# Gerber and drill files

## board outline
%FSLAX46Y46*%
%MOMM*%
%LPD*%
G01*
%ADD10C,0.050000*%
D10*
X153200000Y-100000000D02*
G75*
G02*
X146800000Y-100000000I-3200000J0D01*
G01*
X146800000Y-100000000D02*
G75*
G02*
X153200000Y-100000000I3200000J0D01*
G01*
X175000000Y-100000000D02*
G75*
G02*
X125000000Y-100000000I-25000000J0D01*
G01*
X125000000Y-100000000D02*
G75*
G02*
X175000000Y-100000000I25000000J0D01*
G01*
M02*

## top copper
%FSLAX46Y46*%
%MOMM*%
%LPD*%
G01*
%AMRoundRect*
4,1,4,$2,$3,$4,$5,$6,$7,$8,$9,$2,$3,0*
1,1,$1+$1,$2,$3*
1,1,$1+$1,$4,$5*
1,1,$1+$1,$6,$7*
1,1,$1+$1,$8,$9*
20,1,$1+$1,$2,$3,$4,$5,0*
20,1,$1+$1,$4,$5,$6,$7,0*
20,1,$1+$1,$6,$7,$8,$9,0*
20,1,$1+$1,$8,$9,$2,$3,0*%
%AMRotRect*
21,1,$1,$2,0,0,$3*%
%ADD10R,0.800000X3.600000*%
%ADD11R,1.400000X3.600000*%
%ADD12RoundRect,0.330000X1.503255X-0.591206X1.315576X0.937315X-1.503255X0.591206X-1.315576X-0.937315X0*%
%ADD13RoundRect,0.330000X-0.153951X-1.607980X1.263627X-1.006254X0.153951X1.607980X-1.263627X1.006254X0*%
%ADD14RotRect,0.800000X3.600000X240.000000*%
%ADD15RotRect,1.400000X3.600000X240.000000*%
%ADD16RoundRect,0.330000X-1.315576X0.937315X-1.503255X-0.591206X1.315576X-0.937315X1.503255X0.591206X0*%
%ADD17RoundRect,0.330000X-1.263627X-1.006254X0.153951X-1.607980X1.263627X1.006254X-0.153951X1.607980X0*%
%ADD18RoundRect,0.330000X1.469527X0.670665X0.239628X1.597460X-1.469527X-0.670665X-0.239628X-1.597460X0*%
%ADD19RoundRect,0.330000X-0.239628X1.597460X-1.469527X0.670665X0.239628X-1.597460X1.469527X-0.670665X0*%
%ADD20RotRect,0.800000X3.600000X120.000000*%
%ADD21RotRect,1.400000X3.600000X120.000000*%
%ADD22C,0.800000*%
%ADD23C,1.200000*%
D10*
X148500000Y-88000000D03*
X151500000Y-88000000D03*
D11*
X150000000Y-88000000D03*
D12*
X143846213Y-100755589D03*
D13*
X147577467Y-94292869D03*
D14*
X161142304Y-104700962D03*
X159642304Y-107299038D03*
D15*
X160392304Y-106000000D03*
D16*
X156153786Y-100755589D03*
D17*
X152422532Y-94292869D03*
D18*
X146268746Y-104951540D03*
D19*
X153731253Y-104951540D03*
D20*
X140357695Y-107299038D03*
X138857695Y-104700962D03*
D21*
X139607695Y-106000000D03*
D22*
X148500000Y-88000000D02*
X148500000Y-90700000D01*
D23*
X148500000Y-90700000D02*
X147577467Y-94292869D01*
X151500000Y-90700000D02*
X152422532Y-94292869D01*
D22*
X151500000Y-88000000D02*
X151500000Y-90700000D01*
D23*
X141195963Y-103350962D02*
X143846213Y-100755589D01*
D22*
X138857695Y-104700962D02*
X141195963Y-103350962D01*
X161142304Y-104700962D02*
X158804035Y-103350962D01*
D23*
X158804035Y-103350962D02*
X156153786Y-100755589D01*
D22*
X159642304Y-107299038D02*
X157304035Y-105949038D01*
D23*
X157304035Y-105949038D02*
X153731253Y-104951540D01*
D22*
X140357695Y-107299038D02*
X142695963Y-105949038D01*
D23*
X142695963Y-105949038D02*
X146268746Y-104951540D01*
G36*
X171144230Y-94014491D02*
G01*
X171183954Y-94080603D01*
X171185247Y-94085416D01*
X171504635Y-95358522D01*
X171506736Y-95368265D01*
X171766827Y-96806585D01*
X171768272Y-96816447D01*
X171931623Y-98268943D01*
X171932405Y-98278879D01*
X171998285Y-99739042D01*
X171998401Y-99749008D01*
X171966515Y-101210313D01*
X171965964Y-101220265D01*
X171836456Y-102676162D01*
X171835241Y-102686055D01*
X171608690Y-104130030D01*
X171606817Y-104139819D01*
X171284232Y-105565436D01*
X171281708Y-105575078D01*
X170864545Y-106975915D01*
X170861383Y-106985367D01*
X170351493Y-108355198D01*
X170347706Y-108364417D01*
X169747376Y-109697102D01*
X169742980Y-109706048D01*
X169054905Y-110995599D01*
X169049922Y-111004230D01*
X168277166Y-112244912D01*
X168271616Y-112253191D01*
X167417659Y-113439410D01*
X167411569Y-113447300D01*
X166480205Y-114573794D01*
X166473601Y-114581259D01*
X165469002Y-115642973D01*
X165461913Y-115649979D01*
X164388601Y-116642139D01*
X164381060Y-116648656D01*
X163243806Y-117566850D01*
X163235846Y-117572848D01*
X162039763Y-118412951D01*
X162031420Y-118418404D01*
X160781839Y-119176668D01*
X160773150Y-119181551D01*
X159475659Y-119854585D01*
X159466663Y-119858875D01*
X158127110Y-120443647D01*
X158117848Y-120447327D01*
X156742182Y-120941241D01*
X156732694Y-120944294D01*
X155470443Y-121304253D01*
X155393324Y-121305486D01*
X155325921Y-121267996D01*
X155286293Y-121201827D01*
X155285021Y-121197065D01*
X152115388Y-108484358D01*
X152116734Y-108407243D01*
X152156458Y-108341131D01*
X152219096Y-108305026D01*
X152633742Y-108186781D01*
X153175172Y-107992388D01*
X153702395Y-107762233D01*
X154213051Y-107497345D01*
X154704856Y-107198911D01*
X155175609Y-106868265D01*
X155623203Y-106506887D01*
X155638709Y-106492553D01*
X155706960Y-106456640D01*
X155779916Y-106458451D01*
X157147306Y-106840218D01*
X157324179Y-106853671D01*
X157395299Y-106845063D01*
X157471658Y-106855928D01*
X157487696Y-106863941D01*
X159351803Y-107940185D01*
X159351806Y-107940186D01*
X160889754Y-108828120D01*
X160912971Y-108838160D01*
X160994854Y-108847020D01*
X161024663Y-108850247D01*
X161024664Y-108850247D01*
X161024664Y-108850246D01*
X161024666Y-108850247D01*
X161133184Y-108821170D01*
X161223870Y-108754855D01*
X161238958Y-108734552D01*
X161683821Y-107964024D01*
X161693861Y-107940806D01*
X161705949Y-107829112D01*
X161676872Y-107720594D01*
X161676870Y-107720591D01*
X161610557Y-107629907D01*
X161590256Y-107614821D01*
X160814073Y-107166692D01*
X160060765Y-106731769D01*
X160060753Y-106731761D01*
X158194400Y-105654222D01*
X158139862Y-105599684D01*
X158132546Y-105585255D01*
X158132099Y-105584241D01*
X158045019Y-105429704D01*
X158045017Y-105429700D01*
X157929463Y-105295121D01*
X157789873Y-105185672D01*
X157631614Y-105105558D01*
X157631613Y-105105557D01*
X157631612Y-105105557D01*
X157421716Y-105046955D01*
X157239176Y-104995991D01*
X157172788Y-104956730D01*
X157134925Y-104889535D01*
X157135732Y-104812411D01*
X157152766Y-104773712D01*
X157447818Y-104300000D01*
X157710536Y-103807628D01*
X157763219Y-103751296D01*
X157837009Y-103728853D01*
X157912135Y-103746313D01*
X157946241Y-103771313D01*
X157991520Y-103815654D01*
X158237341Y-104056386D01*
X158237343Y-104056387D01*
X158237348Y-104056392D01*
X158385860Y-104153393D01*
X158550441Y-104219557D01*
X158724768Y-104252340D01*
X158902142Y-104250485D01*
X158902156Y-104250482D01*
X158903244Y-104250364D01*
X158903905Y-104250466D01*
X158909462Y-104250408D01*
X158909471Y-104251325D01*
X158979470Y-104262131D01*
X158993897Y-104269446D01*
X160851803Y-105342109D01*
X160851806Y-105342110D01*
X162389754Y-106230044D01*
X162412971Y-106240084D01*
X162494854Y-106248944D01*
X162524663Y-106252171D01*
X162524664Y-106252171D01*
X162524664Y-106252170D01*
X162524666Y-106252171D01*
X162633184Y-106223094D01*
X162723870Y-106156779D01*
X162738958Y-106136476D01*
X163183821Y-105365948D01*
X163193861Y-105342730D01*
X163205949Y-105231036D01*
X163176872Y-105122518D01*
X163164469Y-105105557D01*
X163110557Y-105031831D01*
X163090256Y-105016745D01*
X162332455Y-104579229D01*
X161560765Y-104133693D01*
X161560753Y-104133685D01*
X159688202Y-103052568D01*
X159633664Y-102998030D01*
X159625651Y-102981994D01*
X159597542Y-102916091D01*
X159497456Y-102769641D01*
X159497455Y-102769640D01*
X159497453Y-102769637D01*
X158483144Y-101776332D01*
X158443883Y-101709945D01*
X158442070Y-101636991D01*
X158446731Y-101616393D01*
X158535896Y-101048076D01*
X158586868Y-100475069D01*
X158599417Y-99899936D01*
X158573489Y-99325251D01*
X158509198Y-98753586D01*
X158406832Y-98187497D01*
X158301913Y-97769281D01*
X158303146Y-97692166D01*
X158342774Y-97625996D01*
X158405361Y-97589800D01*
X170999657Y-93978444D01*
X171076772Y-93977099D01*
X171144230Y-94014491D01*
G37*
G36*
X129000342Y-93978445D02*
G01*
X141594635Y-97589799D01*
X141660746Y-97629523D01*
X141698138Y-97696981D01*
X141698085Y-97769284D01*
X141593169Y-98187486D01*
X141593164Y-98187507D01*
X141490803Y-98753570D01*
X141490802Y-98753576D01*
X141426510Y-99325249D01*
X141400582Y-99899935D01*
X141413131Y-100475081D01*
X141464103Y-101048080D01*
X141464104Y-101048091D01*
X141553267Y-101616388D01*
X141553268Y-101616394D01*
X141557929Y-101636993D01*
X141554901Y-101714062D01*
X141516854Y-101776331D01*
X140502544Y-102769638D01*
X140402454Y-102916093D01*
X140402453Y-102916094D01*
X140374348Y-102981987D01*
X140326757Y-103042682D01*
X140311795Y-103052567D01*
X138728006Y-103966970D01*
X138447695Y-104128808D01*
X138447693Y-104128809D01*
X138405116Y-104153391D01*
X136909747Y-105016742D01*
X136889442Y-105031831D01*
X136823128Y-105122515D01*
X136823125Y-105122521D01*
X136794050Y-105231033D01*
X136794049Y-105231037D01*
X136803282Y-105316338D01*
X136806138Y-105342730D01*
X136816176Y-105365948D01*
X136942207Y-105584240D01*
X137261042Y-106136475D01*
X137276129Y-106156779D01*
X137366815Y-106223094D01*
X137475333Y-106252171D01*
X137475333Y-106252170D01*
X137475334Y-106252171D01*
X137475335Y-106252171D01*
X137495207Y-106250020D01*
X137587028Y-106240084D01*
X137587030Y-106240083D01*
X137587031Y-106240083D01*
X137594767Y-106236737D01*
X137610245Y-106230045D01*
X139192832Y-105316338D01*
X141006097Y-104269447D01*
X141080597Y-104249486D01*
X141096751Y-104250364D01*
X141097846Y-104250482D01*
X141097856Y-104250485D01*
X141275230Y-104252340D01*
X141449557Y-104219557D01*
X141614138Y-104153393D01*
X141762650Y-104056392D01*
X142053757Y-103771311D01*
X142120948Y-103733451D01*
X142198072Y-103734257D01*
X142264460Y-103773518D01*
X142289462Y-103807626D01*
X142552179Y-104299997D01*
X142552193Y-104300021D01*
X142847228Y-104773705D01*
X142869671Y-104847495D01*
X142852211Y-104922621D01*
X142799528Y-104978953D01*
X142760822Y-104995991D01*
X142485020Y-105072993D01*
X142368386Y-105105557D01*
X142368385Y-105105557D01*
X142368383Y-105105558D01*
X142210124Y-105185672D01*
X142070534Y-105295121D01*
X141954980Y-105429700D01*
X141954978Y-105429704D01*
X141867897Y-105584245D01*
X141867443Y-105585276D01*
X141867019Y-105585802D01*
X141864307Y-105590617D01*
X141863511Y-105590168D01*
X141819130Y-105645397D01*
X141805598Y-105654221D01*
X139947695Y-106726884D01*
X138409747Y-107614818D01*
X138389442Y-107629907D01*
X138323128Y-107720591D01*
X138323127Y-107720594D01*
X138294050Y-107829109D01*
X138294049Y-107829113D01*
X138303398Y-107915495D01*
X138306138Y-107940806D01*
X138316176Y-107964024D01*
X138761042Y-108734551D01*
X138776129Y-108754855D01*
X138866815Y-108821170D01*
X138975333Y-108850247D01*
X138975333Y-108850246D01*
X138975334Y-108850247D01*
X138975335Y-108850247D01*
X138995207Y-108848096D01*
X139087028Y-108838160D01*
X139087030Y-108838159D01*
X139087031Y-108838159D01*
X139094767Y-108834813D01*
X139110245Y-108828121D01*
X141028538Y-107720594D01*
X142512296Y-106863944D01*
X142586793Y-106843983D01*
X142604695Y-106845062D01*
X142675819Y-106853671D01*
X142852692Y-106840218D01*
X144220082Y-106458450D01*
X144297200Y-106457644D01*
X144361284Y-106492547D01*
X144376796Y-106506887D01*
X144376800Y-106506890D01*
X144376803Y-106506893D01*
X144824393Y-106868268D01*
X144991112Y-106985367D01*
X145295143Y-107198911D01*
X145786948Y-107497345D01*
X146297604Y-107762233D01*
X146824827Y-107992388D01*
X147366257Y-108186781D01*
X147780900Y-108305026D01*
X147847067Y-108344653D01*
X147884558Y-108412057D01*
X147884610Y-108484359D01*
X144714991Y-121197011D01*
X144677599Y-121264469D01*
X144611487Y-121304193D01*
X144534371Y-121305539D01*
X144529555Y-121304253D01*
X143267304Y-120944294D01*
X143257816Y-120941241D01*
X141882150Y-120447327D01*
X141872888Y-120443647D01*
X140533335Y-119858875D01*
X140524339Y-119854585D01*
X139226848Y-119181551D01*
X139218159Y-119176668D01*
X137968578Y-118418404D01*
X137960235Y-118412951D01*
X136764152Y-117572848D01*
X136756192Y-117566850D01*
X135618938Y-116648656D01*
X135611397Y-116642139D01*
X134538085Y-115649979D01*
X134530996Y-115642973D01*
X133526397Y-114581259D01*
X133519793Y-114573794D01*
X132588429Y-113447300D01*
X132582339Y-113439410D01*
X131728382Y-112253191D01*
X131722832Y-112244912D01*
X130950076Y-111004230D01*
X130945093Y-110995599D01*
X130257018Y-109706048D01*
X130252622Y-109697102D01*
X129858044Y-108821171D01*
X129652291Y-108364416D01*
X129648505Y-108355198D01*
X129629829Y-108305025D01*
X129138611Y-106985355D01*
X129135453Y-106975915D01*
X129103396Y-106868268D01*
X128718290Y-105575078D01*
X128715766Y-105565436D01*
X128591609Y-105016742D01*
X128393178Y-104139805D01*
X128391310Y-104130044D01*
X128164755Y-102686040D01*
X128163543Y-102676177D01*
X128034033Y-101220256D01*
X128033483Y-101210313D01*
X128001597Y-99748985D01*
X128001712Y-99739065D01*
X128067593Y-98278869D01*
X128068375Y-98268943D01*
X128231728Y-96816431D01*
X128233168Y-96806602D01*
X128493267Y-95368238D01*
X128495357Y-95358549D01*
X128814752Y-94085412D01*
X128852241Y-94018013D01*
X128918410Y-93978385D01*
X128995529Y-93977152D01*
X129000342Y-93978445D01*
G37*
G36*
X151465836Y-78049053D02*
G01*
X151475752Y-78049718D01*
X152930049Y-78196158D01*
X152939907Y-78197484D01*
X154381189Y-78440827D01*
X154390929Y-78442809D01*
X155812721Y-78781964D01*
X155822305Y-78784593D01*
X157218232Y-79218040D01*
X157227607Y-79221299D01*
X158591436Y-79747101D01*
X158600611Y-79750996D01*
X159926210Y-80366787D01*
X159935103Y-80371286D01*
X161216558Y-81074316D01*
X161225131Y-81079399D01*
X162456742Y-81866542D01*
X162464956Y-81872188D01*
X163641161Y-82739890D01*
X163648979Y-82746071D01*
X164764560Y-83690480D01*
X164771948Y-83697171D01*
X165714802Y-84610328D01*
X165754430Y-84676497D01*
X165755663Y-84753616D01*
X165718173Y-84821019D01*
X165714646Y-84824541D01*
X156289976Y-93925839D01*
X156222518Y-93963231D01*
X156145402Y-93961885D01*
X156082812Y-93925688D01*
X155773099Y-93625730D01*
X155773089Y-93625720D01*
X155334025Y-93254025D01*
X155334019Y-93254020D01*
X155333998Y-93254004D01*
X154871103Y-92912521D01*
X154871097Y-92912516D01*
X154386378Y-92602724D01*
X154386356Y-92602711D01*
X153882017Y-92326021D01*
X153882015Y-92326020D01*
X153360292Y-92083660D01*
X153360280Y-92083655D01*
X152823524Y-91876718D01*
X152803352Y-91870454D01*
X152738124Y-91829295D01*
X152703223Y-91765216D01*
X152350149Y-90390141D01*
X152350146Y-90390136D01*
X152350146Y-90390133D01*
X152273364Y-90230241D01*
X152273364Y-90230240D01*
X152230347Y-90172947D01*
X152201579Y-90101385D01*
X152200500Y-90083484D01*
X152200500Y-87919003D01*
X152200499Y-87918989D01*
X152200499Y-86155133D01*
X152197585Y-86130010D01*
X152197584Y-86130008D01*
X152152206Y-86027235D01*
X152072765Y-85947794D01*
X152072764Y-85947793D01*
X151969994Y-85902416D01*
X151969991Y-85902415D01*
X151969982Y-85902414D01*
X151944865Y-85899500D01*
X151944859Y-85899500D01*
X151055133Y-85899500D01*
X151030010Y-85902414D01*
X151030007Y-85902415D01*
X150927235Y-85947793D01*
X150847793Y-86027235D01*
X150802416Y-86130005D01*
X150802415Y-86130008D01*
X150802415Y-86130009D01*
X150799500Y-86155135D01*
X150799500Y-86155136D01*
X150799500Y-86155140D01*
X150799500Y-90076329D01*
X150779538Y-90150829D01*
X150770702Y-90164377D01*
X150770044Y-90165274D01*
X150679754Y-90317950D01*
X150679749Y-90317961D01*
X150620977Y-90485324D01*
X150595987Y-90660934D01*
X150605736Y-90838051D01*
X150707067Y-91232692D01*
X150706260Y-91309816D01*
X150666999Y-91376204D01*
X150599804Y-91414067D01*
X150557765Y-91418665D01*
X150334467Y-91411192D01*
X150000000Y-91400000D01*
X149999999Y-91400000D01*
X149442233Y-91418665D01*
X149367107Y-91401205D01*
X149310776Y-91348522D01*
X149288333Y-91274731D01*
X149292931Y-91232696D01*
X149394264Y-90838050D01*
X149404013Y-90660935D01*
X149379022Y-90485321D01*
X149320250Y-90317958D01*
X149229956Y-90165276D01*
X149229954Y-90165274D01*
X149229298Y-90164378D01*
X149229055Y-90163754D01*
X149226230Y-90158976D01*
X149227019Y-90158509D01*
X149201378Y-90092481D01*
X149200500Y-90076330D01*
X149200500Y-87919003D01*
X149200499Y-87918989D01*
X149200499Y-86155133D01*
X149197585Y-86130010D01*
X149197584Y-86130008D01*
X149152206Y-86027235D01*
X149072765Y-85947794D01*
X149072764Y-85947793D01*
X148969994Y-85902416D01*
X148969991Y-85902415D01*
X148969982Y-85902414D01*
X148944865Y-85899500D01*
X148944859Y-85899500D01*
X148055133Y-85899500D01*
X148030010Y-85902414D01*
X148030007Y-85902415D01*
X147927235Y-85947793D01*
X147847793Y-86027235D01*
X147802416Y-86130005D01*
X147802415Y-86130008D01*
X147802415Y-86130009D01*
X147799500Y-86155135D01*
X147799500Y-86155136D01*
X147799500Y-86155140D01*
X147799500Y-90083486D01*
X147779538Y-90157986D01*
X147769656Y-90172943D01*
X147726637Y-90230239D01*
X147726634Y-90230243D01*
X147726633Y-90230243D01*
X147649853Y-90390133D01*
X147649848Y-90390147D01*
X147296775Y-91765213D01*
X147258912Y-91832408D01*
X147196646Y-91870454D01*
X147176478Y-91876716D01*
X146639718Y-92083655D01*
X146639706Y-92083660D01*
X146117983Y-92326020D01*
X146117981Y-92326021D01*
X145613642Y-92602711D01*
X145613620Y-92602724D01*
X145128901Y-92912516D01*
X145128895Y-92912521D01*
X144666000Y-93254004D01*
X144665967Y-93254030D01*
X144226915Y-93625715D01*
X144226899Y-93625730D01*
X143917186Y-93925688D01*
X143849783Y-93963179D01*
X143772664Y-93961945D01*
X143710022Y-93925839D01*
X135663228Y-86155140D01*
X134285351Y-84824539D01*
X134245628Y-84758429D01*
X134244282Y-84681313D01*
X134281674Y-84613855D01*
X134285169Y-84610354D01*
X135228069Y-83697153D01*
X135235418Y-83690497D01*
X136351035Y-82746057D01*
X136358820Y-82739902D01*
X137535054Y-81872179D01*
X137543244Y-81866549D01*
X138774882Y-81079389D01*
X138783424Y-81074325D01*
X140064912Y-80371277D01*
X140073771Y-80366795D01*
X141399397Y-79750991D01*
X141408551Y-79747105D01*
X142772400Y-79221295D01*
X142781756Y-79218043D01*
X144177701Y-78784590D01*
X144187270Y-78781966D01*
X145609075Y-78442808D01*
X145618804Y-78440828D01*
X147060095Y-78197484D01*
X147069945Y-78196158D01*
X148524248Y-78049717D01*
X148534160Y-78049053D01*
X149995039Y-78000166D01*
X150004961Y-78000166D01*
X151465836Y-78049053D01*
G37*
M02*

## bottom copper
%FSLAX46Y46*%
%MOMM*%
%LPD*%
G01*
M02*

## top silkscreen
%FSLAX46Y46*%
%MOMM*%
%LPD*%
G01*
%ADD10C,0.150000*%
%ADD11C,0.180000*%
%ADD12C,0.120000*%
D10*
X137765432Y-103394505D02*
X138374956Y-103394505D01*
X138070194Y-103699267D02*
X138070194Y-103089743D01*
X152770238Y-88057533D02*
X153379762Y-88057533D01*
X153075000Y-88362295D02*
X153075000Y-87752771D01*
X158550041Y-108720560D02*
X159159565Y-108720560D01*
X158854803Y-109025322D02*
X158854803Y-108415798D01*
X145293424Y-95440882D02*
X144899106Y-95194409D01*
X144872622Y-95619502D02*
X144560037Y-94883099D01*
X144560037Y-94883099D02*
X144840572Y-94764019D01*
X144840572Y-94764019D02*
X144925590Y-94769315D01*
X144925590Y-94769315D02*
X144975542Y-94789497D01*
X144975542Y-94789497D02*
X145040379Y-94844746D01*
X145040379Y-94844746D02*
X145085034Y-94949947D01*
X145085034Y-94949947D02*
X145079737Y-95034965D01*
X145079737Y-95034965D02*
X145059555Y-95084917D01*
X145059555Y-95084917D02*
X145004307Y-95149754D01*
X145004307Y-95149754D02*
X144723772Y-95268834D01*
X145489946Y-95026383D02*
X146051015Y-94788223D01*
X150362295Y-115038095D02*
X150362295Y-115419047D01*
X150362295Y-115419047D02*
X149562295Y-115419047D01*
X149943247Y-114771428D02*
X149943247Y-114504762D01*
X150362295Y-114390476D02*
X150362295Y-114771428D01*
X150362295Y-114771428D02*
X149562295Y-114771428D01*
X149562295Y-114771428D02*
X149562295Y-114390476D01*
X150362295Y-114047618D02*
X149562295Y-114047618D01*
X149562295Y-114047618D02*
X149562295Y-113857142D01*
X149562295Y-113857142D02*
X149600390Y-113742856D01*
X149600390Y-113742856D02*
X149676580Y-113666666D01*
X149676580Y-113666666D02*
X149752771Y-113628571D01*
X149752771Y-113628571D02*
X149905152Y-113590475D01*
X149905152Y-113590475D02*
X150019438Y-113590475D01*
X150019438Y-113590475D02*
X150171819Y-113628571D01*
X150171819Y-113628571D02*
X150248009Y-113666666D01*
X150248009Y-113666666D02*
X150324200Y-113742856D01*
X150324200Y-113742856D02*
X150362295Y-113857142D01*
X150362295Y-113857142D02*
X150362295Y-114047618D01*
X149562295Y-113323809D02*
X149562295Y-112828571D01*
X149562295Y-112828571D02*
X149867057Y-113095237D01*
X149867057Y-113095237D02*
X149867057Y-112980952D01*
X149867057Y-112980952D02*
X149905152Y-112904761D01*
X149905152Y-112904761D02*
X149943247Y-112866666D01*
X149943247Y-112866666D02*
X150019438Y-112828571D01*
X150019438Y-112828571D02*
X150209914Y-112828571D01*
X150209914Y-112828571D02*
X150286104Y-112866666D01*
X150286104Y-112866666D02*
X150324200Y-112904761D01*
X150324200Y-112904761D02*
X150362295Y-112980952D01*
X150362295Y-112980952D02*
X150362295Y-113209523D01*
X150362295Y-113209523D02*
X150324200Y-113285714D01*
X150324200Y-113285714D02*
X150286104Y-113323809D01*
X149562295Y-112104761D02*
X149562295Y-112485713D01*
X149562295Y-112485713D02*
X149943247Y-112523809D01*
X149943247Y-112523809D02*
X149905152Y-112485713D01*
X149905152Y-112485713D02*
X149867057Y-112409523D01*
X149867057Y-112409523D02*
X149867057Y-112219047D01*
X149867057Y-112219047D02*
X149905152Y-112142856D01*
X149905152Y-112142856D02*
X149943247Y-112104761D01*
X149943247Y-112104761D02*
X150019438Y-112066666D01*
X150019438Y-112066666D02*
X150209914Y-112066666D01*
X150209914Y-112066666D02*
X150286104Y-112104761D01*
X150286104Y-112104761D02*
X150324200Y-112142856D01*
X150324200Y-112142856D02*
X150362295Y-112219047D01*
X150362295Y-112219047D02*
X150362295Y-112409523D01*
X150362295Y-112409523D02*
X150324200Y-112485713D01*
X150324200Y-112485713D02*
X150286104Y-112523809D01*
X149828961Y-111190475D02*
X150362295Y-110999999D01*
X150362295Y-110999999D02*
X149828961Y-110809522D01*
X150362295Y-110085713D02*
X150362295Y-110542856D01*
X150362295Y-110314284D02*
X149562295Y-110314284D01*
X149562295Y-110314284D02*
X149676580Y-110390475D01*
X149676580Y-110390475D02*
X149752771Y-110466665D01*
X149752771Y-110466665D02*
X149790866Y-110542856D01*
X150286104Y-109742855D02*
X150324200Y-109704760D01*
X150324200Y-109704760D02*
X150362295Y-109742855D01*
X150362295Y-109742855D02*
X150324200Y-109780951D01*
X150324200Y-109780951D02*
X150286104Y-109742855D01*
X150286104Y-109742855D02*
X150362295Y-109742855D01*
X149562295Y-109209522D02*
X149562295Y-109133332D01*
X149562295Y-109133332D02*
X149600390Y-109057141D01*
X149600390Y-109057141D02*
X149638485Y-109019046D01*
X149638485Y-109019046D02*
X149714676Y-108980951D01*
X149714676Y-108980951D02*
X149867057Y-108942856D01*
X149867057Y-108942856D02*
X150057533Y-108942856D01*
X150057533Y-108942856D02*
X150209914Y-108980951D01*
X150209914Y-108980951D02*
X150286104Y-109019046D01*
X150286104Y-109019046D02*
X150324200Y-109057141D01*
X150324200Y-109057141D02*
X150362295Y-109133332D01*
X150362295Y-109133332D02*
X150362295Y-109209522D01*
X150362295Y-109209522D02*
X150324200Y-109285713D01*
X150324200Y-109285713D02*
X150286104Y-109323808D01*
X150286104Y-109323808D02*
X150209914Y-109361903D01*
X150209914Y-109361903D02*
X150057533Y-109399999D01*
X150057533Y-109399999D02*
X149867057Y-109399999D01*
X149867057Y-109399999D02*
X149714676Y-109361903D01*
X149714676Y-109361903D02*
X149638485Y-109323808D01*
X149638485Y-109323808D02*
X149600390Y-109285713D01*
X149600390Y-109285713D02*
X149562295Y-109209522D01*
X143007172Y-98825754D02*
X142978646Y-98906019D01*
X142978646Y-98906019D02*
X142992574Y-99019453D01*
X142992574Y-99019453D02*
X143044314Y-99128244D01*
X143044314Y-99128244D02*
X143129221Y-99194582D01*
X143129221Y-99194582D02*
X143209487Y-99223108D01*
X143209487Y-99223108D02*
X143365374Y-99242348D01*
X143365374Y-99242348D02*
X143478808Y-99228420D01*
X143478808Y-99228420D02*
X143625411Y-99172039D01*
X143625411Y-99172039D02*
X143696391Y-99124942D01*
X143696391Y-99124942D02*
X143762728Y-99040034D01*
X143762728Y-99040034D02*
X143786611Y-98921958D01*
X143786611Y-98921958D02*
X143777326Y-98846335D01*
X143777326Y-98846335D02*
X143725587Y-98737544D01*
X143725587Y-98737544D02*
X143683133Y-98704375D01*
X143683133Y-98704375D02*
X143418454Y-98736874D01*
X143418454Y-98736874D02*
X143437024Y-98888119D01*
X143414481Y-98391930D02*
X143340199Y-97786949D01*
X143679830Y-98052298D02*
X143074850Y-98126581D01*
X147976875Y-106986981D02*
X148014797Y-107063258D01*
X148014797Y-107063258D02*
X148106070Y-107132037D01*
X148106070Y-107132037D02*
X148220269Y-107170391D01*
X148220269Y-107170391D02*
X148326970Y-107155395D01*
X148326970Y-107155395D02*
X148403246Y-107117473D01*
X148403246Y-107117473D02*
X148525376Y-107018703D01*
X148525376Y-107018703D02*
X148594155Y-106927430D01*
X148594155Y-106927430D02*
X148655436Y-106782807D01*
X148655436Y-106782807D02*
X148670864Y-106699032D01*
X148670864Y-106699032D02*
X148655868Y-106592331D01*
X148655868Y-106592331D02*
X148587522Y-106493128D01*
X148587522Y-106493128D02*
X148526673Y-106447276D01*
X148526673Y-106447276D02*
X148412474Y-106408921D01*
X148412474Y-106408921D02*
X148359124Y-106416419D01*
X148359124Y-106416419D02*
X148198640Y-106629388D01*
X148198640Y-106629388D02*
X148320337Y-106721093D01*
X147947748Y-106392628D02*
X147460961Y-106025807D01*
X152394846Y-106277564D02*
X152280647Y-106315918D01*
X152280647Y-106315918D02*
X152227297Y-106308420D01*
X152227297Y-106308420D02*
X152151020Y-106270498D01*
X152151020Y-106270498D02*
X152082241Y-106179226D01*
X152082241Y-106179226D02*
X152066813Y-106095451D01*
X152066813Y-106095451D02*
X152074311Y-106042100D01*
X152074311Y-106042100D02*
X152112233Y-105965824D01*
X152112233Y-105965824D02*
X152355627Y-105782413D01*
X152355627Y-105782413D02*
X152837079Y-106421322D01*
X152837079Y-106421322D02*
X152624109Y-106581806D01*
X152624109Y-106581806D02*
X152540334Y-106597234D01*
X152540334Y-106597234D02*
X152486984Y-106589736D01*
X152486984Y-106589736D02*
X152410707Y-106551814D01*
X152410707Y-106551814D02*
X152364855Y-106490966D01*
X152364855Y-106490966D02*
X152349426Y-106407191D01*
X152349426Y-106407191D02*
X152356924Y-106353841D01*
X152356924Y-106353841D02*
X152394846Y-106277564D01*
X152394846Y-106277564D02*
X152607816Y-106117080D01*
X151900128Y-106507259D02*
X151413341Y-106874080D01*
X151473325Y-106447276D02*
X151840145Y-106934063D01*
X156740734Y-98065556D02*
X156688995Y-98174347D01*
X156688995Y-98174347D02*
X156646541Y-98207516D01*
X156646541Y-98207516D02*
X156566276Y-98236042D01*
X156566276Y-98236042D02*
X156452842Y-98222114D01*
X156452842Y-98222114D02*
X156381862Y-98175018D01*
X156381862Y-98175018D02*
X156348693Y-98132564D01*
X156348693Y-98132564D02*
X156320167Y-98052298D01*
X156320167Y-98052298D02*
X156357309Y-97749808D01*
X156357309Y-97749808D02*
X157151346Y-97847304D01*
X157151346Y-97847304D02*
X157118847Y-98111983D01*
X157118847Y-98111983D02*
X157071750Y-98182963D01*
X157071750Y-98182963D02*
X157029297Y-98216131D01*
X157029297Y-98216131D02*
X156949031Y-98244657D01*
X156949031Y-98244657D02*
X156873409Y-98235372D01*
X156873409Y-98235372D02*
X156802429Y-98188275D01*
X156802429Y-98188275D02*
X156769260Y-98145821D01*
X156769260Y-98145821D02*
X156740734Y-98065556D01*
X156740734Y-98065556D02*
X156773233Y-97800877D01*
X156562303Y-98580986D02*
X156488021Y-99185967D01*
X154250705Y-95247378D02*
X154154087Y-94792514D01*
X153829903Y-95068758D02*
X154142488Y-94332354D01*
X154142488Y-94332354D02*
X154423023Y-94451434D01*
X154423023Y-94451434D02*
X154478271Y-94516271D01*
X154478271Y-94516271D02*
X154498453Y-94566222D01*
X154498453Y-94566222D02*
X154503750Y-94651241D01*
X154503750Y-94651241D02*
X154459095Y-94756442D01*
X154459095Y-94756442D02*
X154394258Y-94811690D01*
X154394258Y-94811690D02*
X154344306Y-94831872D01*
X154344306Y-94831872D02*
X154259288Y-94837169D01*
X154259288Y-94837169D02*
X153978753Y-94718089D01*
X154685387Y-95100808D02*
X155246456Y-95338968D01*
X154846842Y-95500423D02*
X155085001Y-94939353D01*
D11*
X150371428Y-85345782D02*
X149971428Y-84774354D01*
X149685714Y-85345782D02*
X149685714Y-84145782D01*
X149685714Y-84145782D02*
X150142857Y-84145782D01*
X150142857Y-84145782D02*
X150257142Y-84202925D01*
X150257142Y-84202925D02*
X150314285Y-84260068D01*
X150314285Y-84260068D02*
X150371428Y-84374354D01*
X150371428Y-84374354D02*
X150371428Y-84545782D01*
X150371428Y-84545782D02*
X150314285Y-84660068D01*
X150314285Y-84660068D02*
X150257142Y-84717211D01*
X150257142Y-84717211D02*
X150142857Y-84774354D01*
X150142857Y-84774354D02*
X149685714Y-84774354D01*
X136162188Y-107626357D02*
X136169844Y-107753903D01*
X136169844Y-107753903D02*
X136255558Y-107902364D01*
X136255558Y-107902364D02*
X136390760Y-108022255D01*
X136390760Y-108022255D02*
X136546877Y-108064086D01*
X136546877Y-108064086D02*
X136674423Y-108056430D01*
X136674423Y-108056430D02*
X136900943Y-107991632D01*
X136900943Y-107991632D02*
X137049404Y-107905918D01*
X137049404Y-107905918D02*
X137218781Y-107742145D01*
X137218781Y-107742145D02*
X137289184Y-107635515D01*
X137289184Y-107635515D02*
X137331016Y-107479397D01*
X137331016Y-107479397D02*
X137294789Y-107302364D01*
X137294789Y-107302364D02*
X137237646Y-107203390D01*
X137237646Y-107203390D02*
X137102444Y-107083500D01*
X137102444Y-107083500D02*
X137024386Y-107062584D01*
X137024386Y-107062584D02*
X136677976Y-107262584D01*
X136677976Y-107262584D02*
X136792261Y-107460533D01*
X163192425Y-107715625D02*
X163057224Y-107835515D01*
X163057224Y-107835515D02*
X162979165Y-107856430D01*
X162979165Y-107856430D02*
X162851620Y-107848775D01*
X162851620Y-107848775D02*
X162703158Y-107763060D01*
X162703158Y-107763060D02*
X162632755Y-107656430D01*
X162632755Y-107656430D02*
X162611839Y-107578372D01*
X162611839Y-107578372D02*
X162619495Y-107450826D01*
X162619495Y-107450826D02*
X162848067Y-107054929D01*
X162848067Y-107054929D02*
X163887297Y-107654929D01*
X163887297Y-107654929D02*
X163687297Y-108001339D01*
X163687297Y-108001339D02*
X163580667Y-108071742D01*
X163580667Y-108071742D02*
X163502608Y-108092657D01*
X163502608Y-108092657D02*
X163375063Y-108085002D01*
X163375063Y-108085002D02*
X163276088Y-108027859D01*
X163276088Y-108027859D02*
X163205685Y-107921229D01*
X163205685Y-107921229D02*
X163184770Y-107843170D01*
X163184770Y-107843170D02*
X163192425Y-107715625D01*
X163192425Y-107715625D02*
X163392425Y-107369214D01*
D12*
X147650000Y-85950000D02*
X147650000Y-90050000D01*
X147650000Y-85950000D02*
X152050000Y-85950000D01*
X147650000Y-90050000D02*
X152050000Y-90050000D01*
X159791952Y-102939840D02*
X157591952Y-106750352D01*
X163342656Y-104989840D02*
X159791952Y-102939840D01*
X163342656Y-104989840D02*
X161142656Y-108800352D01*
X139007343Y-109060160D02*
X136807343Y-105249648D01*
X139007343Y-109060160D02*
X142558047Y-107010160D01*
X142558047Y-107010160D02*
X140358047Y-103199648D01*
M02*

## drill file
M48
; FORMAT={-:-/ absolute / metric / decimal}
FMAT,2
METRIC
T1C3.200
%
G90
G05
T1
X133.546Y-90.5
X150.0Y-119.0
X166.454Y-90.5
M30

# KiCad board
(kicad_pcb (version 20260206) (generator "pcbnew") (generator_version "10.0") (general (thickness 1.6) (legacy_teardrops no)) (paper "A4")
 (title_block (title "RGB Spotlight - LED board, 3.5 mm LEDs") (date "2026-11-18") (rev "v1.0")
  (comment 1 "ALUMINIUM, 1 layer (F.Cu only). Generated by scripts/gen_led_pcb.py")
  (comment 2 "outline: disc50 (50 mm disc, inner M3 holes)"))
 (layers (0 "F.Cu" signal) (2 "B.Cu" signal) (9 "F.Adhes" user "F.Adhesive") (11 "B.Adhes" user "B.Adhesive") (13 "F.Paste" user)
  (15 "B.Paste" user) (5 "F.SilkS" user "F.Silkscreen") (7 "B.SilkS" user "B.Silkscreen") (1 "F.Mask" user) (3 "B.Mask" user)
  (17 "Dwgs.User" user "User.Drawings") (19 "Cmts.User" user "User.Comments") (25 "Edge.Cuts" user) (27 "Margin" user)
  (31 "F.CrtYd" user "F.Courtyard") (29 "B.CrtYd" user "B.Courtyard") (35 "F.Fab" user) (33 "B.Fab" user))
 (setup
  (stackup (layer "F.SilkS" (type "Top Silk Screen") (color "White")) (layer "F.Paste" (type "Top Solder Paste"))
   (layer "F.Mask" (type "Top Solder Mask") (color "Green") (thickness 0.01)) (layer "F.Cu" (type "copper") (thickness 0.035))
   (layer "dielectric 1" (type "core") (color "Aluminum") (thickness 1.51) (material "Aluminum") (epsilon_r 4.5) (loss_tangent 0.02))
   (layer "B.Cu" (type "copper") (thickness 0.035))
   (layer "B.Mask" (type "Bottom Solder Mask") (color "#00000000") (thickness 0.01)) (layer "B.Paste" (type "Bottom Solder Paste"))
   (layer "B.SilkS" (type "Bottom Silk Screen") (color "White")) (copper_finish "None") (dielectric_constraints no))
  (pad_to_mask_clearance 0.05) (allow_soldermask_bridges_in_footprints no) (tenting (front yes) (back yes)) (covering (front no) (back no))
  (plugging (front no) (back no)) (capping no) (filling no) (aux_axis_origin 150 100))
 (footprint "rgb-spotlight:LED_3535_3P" (layer "F.Cu") (at 150 88)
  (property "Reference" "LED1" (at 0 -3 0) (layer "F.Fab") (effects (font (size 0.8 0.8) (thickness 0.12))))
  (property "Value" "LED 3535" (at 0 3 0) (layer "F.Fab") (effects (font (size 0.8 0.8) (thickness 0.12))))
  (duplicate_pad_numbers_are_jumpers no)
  (fp_line (start -2.35 -2.05) (end -2.35 2.05) (stroke (width 0.12) (type solid)) (layer "F.SilkS"))
  (fp_line (start -2.35 -2.05) (end 2.05 -2.05) (stroke (width 0.12) (type solid)) (layer "F.SilkS"))
  (fp_line (start -2.35 2.05) (end 2.05 2.05) (stroke (width 0.12) (type solid)) (layer "F.SilkS"))
  (pad "1" smd rect (at -1.5 0) (size 0.8 3.6) (layers "F.Cu" "F.Mask" "F.Paste") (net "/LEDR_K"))
  (pad "2" smd rect (at 1.5 0) (size 0.8 3.6) (layers "F.Cu" "F.Mask" "F.Paste") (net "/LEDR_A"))
  (pad "3" smd rect (at 0 0) (size 1.4 3.6) (layers "F.Cu" "F.Mask" "F.Paste") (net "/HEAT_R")))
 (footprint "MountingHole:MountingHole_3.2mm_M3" (layer "F.Cu") (at 166.454482 90.5)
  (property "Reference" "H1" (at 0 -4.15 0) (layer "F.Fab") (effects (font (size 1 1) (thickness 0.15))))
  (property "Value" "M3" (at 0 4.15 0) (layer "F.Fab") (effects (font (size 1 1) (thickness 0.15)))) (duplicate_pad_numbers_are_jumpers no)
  (pad "" np_thru_hole circle (at 0 0) (size 3.2 3.2) (drill 3.2) (layers "*.Cu" "*.Mask")))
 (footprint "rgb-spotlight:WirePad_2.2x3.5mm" (layer "F.Cu") (at 143.846213 100.755589 97)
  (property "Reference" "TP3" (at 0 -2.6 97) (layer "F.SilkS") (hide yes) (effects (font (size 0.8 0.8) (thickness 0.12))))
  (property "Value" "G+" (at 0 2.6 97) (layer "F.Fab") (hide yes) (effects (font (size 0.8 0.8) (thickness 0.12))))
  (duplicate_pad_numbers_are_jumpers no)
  (pad "1" smd roundrect (at 0 0 97) (size 2.2 3.5) (layers "F.Cu" "F.Mask") (roundrect_rratio 0.15) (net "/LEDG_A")))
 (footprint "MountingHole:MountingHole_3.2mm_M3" (layer "F.Cu") (at 150 119)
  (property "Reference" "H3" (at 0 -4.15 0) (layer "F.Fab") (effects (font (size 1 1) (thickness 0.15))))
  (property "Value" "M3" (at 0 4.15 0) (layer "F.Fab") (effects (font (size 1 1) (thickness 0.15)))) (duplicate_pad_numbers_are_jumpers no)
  (pad "" np_thru_hole circle (at 0 0) (size 3.2 3.2) (drill 3.2) (layers "*.Cu" "*.Mask")))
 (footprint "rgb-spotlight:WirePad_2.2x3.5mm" (layer "F.Cu") (at 147.577467 94.292869 23)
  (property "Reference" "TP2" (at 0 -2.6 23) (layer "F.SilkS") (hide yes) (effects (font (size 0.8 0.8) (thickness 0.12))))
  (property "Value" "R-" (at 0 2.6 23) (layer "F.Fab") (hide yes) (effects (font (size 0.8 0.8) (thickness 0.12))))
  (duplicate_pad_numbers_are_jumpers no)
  (pad "1" smd roundrect (at 0 0 23) (size 2.2 3.5) (layers "F.Cu" "F.Mask") (roundrect_rratio 0.15) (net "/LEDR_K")))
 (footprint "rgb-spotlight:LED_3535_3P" (layer "F.Cu") (at 160.392304 106 -120)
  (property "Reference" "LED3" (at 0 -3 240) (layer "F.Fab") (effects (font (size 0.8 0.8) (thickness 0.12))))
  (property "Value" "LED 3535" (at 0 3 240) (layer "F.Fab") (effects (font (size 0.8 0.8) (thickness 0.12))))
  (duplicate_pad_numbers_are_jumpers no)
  (fp_line (start -2.35 2.05) (end 2.05 2.05) (stroke (width 0.12) (type solid)) (layer "F.SilkS"))
  (fp_line (start -2.35 -2.05) (end -2.35 2.05) (stroke (width 0.12) (type solid)) (layer "F.SilkS"))
  (fp_line (start -2.35 -2.05) (end 2.05 -2.05) (stroke (width 0.12) (type solid)) (layer "F.SilkS"))
  (pad "1" smd rect (at -1.5 0 240) (size 0.8 3.6) (layers "F.Cu" "F.Mask" "F.Paste") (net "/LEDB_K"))
  (pad "2" smd rect (at 1.5 0 240) (size 0.8 3.6) (layers "F.Cu" "F.Mask" "F.Paste") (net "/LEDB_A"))
  (pad "3" smd rect (at 0 0 240) (size 1.4 3.6) (layers "F.Cu" "F.Mask" "F.Paste") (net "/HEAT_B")))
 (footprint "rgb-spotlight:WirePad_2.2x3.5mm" (layer "F.Cu") (at 156.153786 100.755589 -97)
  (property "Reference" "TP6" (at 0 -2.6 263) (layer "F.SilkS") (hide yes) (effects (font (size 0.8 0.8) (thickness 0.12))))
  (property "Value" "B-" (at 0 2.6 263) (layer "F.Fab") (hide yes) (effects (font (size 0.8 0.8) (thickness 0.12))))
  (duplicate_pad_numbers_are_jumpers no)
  (pad "1" smd roundrect (at 0 0 263) (size 2.2 3.5) (layers "F.Cu" "F.Mask") (roundrect_rratio 0.15) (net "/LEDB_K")))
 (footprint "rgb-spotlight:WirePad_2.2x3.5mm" (layer "F.Cu") (at 152.422532 94.292869 -23)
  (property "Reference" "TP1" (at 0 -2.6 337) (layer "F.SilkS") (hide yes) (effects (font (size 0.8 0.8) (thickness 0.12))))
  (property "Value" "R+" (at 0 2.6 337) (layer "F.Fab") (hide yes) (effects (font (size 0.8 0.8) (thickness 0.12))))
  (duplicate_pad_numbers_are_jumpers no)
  (pad "1" smd roundrect (at 0 0 337) (size 2.2 3.5) (layers "F.Cu" "F.Mask") (roundrect_rratio 0.15) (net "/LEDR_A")))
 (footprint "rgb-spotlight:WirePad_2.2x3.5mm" (layer "F.Cu") (at 146.268746 104.95154 143)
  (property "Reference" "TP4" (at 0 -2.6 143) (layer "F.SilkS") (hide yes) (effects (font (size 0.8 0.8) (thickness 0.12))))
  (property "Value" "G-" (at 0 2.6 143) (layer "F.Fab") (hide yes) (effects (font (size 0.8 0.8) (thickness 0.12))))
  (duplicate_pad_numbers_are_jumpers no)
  (pad "1" smd roundrect (at 0 0 143) (size 2.2 3.5) (layers "F.Cu" "F.Mask") (roundrect_rratio 0.15) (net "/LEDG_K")))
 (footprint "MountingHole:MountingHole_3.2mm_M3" (layer "F.Cu") (at 133.545517 90.5)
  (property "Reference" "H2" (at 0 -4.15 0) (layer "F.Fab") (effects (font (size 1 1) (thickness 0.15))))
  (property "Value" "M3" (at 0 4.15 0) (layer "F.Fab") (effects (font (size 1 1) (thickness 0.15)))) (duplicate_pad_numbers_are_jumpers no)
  (pad "" np_thru_hole circle (at 0 0) (size 3.2 3.2) (drill 3.2) (layers "*.Cu" "*.Mask")))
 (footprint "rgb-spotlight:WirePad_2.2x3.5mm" (layer "F.Cu") (at 153.731253 104.95154 -143)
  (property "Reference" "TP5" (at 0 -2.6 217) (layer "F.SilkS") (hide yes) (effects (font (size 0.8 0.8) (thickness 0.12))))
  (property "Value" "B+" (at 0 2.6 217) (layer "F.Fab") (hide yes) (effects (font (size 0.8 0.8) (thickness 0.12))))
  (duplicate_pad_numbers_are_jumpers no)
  (pad "1" smd roundrect (at 0 0 217) (size 2.2 3.5) (layers "F.Cu" "F.Mask") (roundrect_rratio 0.15) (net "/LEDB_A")))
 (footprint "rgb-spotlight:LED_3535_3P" (layer "F.Cu") (at 139.607695 106 120)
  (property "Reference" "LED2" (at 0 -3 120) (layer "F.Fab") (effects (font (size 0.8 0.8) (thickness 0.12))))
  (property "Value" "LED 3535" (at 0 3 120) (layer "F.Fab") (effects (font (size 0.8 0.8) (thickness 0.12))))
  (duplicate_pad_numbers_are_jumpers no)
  (fp_line (start -2.35 -2.05) (end 2.05 -2.05) (stroke (width 0.12) (type solid)) (layer "F.SilkS"))
  (fp_line (start -2.35 -2.05) (end -2.35 2.05) (stroke (width 0.12) (type solid)) (layer "F.SilkS"))
  (fp_line (start -2.35 2.05) (end 2.05 2.05) (stroke (width 0.12) (type solid)) (layer "F.SilkS"))
  (pad "1" smd rect (at -1.5 0 120) (size 0.8 3.6) (layers "F.Cu" "F.Mask" "F.Paste") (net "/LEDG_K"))
  (pad "2" smd rect (at 1.5 0 120) (size 0.8 3.6) (layers "F.Cu" "F.Mask" "F.Paste") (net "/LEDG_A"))
  (pad "3" smd rect (at 0 0 120) (size 1.4 3.6) (layers "F.Cu" "F.Mask" "F.Paste") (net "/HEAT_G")))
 (gr_circle (center 150 100) (end 153.2 100) (stroke (width 0.05) (type default)) (fill no) (layer "Edge.Cuts"))
 (gr_circle (center 150 100) (end 175 100) (stroke (width 0.05) (type default)) (fill no) (layer "Edge.Cuts"))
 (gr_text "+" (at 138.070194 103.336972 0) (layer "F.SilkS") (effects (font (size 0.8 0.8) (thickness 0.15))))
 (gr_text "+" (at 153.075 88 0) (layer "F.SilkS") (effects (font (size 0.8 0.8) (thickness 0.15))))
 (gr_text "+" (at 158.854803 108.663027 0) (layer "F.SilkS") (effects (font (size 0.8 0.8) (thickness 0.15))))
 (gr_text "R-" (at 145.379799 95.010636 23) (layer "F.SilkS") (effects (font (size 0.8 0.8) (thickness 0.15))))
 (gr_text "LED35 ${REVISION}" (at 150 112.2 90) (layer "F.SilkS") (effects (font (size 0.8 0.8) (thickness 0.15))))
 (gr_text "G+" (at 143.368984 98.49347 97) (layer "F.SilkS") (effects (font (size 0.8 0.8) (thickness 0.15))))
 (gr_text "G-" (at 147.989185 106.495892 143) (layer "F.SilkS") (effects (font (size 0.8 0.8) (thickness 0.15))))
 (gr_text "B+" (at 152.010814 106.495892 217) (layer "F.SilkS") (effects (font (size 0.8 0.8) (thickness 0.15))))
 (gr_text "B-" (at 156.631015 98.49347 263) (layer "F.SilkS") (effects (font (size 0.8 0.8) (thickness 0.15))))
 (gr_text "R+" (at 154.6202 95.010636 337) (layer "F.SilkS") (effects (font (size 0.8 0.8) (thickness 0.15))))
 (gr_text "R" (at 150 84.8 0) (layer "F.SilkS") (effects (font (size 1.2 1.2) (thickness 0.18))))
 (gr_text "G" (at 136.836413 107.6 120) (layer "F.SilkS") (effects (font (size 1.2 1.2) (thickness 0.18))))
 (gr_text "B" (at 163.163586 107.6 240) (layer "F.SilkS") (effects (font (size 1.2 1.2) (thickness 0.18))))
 (segment (start 148.5 88) (end 148.5 90.7) (width 0.8) (layer "F.Cu") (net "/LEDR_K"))
 (segment (start 148.5 90.7) (end 147.577467 94.292869) (width 1.2) (layer "F.Cu") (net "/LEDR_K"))
 (segment (start 151.5 90.7) (end 152.422532 94.292869) (width 1.2) (layer "F.Cu") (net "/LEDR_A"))
 (segment (start 151.5 88) (end 151.5 90.7) (width 0.8) (layer "F.Cu") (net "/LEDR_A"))
 (segment (start 141.195963 103.350962) (end 143.846213 100.755589) (width 1.2) (layer "F.Cu") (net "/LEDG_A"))
 (segment (start 138.857695 104.700962) (end 141.195963 103.350962) (width 0.8) (layer "F.Cu") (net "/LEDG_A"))
 (segment (start 161.142304 104.700962) (end 158.804035 103.350962) (width 0.8) (layer "F.Cu") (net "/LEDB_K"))
 (segment (start 158.804035 103.350962) (end 156.153786 100.755589) (width 1.2) (layer "F.Cu") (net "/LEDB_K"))
 (segment (start 159.642304 107.299038) (end 157.304035 105.949038) (width 0.8) (layer "F.Cu") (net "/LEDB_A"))
 (segment (start 157.304035 105.949038) (end 153.731253 104.95154) (width 1.2) (layer "F.Cu") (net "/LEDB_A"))
 (segment (start 140.357695 107.299038) (end 142.695963 105.949038) (width 0.8) (layer "F.Cu") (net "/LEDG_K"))
 (segment (start 142.695963 105.949038) (end 146.268746 104.95154) (width 1.2) (layer "F.Cu") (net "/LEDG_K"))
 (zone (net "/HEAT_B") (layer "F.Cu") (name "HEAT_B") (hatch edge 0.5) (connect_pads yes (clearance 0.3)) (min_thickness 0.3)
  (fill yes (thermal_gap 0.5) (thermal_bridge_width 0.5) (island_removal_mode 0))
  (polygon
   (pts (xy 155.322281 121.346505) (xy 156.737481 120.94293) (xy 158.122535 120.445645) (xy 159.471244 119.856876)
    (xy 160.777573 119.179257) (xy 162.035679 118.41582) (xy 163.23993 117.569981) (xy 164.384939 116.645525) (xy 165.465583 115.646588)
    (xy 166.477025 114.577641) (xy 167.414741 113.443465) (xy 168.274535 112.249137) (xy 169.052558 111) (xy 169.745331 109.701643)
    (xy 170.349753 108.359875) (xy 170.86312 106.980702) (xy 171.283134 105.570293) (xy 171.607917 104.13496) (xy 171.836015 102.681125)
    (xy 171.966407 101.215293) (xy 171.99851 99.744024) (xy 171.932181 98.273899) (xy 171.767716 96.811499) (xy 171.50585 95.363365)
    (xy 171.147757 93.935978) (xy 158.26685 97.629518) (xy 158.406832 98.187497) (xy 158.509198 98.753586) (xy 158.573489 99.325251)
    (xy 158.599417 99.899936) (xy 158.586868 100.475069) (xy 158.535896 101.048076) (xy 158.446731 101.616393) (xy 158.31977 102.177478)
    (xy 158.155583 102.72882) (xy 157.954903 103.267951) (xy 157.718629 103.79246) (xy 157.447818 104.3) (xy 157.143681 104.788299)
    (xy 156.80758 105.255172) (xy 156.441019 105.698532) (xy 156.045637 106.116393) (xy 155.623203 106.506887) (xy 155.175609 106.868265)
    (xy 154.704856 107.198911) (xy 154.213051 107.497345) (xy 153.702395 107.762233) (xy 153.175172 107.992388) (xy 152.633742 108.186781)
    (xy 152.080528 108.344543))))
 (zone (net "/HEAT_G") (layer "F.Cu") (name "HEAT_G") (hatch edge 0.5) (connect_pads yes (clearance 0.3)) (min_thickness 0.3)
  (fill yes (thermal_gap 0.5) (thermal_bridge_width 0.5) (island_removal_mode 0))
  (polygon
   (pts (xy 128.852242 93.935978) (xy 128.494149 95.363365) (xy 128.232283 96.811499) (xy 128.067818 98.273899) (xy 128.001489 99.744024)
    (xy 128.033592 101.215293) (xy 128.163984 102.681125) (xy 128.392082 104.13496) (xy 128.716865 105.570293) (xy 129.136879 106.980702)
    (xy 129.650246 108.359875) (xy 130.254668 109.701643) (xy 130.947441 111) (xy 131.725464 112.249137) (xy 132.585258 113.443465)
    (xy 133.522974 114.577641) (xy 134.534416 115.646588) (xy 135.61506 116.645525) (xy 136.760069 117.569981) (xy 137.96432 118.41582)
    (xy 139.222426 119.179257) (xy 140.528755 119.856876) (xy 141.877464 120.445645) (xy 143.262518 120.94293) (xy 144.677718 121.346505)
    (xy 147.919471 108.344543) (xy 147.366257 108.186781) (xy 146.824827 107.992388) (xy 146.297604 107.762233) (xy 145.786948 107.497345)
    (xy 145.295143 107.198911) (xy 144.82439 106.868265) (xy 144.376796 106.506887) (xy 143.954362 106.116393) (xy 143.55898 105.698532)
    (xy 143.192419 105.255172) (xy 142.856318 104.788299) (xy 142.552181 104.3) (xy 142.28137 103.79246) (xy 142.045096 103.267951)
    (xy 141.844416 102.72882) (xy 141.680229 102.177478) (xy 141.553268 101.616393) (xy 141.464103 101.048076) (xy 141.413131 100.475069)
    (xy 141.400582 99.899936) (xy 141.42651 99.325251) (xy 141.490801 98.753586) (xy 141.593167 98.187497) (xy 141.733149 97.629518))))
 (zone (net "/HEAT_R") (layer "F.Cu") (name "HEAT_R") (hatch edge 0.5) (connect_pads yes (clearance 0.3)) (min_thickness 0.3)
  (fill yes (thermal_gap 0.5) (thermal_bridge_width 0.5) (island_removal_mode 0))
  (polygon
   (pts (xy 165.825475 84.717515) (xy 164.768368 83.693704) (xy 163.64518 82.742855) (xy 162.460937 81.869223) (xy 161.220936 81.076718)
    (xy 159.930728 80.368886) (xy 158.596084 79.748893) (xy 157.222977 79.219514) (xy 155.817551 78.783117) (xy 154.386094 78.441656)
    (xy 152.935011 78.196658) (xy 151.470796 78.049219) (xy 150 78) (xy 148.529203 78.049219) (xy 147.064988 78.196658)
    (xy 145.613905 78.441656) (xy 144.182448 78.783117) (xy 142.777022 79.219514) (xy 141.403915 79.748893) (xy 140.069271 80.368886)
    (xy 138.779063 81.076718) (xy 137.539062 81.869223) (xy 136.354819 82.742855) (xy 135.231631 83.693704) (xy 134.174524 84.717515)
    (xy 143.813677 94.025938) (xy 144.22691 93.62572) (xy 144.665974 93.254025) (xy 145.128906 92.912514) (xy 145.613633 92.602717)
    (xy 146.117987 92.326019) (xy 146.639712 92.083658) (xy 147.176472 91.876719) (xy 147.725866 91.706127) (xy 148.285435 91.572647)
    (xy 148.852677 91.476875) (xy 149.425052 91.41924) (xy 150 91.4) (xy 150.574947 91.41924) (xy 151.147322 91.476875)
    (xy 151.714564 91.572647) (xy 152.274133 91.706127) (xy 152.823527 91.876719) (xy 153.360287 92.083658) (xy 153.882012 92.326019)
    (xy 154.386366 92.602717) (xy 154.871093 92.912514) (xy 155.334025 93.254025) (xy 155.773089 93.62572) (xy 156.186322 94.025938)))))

